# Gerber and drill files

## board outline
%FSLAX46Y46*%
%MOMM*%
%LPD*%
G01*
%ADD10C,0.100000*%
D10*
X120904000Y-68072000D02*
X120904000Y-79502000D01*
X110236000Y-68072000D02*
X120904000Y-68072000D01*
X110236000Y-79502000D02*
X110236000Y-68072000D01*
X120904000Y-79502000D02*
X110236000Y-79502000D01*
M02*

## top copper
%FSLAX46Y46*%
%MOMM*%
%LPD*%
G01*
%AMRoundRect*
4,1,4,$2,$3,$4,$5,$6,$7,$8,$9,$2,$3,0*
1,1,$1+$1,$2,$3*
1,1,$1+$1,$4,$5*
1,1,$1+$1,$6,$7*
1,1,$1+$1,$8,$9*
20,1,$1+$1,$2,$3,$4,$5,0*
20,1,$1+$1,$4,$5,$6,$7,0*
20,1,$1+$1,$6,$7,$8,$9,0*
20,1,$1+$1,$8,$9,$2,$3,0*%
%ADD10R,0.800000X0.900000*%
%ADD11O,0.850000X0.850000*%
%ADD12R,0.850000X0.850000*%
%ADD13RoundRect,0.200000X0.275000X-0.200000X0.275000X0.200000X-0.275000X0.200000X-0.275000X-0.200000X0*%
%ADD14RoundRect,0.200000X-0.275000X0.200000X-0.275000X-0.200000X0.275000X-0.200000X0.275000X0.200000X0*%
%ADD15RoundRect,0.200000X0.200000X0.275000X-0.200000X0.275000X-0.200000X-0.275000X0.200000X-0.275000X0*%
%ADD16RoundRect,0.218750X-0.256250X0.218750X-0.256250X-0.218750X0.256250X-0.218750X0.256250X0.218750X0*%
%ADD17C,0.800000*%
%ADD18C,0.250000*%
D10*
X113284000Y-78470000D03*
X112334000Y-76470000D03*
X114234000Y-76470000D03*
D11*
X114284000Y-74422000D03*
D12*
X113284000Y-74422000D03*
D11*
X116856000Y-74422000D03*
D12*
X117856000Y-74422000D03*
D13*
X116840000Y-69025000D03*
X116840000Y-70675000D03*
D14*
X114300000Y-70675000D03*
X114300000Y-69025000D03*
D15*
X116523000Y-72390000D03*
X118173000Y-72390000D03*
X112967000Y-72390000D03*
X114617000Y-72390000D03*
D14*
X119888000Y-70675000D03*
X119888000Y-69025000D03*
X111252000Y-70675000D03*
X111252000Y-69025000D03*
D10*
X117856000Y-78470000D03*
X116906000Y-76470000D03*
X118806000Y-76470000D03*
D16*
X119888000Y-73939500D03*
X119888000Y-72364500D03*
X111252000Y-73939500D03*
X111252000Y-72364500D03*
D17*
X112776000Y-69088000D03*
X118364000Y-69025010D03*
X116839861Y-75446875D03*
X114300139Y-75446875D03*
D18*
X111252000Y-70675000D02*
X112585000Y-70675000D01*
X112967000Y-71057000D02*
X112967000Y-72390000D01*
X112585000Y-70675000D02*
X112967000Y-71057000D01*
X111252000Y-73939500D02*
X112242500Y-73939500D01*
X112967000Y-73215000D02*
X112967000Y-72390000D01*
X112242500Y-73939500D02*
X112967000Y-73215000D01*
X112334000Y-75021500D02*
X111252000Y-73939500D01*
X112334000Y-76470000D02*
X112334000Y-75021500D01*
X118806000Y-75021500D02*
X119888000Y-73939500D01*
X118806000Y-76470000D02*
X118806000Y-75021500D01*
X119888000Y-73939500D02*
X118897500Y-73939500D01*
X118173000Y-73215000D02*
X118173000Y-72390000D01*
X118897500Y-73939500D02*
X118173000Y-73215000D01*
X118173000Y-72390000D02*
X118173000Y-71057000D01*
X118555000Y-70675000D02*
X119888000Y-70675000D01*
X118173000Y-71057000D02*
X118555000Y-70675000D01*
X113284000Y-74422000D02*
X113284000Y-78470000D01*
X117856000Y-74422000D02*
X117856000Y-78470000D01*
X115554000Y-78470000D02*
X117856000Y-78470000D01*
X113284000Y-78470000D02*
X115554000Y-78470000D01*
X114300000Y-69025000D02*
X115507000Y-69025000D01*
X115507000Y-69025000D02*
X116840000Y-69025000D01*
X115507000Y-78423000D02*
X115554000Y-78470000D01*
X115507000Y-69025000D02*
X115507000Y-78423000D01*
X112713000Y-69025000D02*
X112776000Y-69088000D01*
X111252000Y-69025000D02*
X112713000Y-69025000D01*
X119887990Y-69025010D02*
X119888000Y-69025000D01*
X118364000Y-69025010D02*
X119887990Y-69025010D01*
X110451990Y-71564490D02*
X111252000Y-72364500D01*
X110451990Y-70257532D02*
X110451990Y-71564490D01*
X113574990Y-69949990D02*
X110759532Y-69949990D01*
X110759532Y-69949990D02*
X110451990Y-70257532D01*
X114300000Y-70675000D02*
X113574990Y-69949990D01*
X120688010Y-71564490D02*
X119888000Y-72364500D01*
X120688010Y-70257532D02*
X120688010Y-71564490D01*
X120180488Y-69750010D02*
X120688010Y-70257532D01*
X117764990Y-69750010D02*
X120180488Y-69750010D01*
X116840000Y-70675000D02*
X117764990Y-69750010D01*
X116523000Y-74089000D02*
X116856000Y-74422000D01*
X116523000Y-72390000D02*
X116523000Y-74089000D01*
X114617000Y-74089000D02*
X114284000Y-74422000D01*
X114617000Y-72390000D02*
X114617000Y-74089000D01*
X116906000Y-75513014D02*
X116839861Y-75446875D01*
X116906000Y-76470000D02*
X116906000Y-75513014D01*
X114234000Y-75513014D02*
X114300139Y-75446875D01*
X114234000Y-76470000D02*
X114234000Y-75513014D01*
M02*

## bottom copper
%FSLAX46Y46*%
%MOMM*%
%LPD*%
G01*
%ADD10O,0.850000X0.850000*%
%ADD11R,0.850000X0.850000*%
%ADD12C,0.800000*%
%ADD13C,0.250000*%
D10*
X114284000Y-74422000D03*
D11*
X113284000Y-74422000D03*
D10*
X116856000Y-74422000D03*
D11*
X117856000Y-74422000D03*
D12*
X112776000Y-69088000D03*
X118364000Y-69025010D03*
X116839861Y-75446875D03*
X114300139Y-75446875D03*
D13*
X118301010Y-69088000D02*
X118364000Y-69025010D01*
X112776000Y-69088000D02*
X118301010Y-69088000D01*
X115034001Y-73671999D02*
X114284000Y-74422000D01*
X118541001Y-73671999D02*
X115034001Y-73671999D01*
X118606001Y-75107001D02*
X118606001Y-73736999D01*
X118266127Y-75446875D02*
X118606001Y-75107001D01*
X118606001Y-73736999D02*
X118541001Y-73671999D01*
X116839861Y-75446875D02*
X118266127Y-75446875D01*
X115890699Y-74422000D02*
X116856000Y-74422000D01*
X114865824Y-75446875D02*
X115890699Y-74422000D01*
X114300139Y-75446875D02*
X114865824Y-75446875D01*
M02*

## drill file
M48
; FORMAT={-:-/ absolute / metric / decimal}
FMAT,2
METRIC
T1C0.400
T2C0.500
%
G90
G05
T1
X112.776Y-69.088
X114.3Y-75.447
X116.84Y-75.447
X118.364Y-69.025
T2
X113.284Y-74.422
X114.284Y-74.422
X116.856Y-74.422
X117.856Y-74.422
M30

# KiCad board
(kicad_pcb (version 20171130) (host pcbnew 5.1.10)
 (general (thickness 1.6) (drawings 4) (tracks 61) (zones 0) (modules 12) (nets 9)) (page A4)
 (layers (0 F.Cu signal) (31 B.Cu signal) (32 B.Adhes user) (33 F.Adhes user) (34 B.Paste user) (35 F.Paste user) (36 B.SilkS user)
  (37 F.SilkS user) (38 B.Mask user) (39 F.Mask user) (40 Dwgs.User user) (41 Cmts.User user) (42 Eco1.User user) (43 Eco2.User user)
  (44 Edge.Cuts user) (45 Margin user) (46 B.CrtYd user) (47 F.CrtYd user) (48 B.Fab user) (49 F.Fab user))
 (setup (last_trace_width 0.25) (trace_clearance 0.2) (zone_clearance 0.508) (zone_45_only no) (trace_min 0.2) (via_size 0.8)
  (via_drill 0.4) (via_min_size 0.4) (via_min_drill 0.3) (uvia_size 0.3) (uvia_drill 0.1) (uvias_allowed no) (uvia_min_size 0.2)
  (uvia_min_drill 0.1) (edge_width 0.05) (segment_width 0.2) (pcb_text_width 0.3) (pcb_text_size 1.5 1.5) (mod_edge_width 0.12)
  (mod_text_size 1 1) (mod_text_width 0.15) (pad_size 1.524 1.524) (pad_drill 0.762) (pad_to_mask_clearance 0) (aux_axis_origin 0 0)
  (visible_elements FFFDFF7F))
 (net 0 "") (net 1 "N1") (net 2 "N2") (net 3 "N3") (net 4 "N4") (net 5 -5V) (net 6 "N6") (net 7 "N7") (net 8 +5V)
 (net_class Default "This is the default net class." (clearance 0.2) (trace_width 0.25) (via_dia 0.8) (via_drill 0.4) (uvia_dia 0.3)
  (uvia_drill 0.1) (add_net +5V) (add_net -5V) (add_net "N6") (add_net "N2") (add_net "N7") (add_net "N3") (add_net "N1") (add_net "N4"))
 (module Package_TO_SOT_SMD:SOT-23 (layer F.Cu) (at 113.284 77.47 270)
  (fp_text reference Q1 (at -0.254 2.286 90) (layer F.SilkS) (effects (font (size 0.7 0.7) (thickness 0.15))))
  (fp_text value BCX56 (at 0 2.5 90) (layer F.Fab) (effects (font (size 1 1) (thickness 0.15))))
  (pad 3 smd rect (at 1 0 270) (size 0.9 0.8) (layers F.Cu F.Paste F.Mask) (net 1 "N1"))
  (pad 2 smd rect (at -1 0.95 270) (size 0.9 0.8) (layers F.Cu F.Paste F.Mask) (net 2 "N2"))
  (pad 1 smd rect (at -1 -0.95 270) (size 0.9 0.8) (layers F.Cu F.Paste F.Mask) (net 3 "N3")))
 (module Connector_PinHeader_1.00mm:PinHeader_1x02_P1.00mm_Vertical (layer F.Cu) (at 113.284 74.422 90)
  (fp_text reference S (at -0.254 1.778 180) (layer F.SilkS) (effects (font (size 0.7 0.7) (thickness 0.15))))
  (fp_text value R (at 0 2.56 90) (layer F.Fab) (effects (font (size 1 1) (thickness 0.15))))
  (pad 2 thru_hole oval (at 0 1 90) (size 0.85 0.85) (drill 0.5) (layers *.Cu *.Mask) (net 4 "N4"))
  (pad 1 thru_hole rect (at 0 0 90) (size 0.85 0.85) (drill 0.5) (layers *.Cu *.Mask) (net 1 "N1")))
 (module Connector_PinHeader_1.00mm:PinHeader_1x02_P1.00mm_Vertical (layer F.Cu) (at 117.856 74.422 270)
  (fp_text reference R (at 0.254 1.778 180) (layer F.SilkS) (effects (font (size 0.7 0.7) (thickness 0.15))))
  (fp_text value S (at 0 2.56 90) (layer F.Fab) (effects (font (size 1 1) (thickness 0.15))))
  (pad 2 thru_hole oval (at 0 1 270) (size 0.85 0.85) (drill 0.5) (layers *.Cu *.Mask) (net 3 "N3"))
  (pad 1 thru_hole rect (at 0 0 270) (size 0.85 0.85) (drill 0.5) (layers *.Cu *.Mask) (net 1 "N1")))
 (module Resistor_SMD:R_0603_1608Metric (layer F.Cu) (at 116.84 69.85 90)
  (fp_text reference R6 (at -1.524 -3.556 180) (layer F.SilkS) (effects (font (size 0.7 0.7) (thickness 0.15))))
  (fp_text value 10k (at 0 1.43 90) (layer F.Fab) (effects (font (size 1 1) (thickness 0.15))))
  (pad 2 smd roundrect (at 0.825 0 90) (size 0.8 0.95) (layers F.Cu F.Paste F.Mask) (roundrect_rratio 0.25) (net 1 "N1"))
  (pad 1 smd roundrect (at -0.825 0 90) (size 0.8 0.95) (layers F.Cu F.Paste F.Mask) (roundrect_rratio 0.25) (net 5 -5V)))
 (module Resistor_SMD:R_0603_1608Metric (layer F.Cu) (at 114.3 69.85 270)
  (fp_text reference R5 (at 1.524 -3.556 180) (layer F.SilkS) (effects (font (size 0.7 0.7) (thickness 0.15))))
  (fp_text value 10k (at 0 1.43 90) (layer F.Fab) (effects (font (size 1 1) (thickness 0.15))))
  (pad 2 smd roundrect (at 0.825 0 270) (size 0.8 0.95) (layers F.Cu F.Paste F.Mask) (roundrect_rratio 0.25) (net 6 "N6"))
  (pad 1 smd roundrect (at -0.825 0 270) (size 0.8 0.95) (layers F.Cu F.Paste F.Mask) (roundrect_rratio 0.25) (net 1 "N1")))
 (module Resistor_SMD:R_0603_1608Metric (layer F.Cu) (at 117.348 72.39 180)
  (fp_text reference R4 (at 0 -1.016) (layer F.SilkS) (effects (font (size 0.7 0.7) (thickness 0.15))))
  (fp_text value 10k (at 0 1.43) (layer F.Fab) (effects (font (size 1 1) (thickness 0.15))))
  (pad 2 smd roundrect (at 0.825 0 180) (size 0.8 0.95) (layers F.Cu F.Paste F.Mask) (roundrect_rratio 0.25) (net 3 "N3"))
  (pad 1 smd roundrect (at -0.825 0 180) (size 0.8 0.95) (layers F.Cu F.Paste F.Mask) (roundrect_rratio 0.25) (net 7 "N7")))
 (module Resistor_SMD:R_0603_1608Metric (layer F.Cu) (at 113.792 72.39 180)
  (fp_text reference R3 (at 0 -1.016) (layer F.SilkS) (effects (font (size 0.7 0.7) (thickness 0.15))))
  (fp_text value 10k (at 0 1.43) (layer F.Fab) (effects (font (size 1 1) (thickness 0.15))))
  (pad 2 smd roundrect (at 0.825 0 180) (size 0.8 0.95) (layers F.Cu F.Paste F.Mask) (roundrect_rratio 0.25) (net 2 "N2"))
  (pad 1 smd roundrect (at -0.825 0 180) (size 0.8 0.95) (layers F.Cu F.Paste F.Mask) (roundrect_rratio 0.25) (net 4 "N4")))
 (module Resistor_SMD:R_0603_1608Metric (layer F.Cu) (at 119.888 69.85 270)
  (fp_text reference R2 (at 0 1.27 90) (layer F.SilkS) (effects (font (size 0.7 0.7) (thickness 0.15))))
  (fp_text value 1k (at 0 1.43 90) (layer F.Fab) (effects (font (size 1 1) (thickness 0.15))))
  (pad 2 smd roundrect (at 0.825 0 270) (size 0.8 0.95) (layers F.Cu F.Paste F.Mask) (roundrect_rratio 0.25) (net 7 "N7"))
  (pad 1 smd roundrect (at -0.825 0 270) (size 0.8 0.95) (layers F.Cu F.Paste F.Mask) (roundrect_rratio 0.25) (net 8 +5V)))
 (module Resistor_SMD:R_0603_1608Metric (layer F.Cu) (at 111.252 69.85 270)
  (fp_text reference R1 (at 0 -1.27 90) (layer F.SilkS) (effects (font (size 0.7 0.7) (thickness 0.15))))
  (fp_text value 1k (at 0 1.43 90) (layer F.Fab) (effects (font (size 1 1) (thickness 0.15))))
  (pad 2 smd roundrect (at 0.825 0 270) (size 0.8 0.95) (layers F.Cu F.Paste F.Mask) (roundrect_rratio 0.25) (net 2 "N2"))
  (pad 1 smd roundrect (at -0.825 0 270) (size 0.8 0.95) (layers F.Cu F.Paste F.Mask) (roundrect_rratio 0.25) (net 8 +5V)))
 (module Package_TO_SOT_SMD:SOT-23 (layer F.Cu) (at 117.856 77.47 270)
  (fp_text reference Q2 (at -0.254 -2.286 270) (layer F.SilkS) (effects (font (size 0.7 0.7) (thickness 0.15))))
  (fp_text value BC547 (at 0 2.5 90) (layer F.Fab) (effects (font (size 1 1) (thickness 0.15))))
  (pad 3 smd rect (at 1 0 270) (size 0.9 0.8) (layers F.Cu F.Paste F.Mask) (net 1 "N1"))
  (pad 2 smd rect (at -1 0.95 270) (size 0.9 0.8) (layers F.Cu F.Paste F.Mask) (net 4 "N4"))
  (pad 1 smd rect (at -1 -0.95 270) (size 0.9 0.8) (layers F.Cu F.Paste F.Mask) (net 7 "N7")))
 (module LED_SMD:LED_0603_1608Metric (layer F.Cu) (at 119.888 73.152 270)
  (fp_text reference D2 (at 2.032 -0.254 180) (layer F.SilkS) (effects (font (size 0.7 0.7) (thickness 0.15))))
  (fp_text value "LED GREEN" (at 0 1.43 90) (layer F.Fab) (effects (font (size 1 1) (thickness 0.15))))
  (pad 2 smd roundrect (at 0.7875 0 270) (size 0.875 0.95) (layers F.Cu F.Paste F.Mask) (roundrect_rratio 0.25) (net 7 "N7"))
  (pad 1 smd roundrect (at -0.7875 0 270) (size 0.875 0.95) (layers F.Cu F.Paste F.Mask) (roundrect_rratio 0.25) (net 5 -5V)))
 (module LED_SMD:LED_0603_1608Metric (layer F.Cu) (at 111.252 73.152 270)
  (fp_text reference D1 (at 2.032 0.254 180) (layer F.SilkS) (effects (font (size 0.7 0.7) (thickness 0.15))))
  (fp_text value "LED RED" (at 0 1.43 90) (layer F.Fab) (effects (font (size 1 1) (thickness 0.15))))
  (pad 2 smd roundrect (at 0.7875 0 270) (size 0.875 0.95) (layers F.Cu F.Paste F.Mask) (roundrect_rratio 0.25) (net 2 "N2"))
  (pad 1 smd roundrect (at -0.7875 0 270) (size 0.875 0.95) (layers F.Cu F.Paste F.Mask) (roundrect_rratio 0.25) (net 6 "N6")))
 (gr_line (start 120.904 68.072) (end 120.904 79.502) (layer Edge.Cuts) (width 0.1))
 (gr_line (start 110.236 68.072) (end 120.904 68.072) (layer Edge.Cuts) (width 0.1))
 (gr_line (start 110.236 79.502) (end 110.236 68.072) (layer Edge.Cuts) (width 0.1))
 (gr_line (start 120.904 79.502) (end 110.236 79.502) (layer Edge.Cuts) (width 0.1))
 (segment (start 111.252 70.675) (end 112.585 70.675) (width 0.25) (layer F.Cu) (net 2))
 (segment (start 112.967 71.057) (end 112.967 72.39) (width 0.25) (layer F.Cu) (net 2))
 (segment (start 112.585 70.675) (end 112.967 71.057) (width 0.25) (layer F.Cu) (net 2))
 (segment (start 111.252 73.9395) (end 112.2425 73.9395) (width 0.25) (layer F.Cu) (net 2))
 (segment (start 112.967 73.215) (end 112.967 72.39) (width 0.25) (layer F.Cu) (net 2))
 (segment (start 112.2425 73.9395) (end 112.967 73.215) (width 0.25) (layer F.Cu) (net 2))
 (segment (start 112.334 75.0215) (end 111.252 73.9395) (width 0.25) (layer F.Cu) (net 2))
 (segment (start 112.334 76.47) (end 112.334 75.0215) (width 0.25) (layer F.Cu) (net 2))
 (segment (start 118.806 75.0215) (end 119.888 73.9395) (width 0.25) (layer F.Cu) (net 7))
 (segment (start 118.806 76.47) (end 118.806 75.0215) (width 0.25) (layer F.Cu) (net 7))
 (segment (start 119.888 73.9395) (end 118.8975 73.9395) (width 0.25) (layer F.Cu) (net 7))
 (segment (start 118.173 73.215) (end 118.173 72.39) (width 0.25) (layer F.Cu) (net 7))
 (segment (start 118.8975 73.9395) (end 118.173 73.215) (width 0.25) (layer F.Cu) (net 7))
 (segment (start 118.173 72.39) (end 118.173 71.057) (width 0.25) (layer F.Cu) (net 7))
 (segment (start 118.555 70.675) (end 119.888 70.675) (width 0.25) (layer F.Cu) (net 7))
 (segment (start 118.173 71.057) (end 118.555 70.675) (width 0.25) (layer F.Cu) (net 7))
 (segment (start 113.284 74.422) (end 113.284 78.47) (width 0.25) (layer F.Cu) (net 1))
 (segment (start 117.856 74.422) (end 117.856 78.47) (width 0.25) (layer F.Cu) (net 1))
 (segment (start 115.554 78.47) (end 117.856 78.47) (width 0.25) (layer F.Cu) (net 1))
 (segment (start 113.284 78.47) (end 115.554 78.47) (width 0.25) (layer F.Cu) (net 1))
 (segment (start 114.3 69.025) (end 115.507 69.025) (width 0.25) (layer F.Cu) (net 1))
 (segment (start 115.507 69.025) (end 116.84 69.025) (width 0.25) (layer F.Cu) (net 1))
 (segment (start 115.507 78.423) (end 115.554 78.47) (width 0.25) (layer F.Cu) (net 1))
 (segment (start 115.507 69.025) (end 115.507 78.423) (width 0.25) (layer F.Cu) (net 1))
 (via (at 112.776 69.088) (size 0.8) (drill 0.4) (layers F.Cu B.Cu) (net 8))
 (segment (start 112.713 69.025) (end 112.776 69.088) (width 0.25) (layer F.Cu) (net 8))
 (segment (start 111.252 69.025) (end 112.713 69.025) (width 0.25) (layer F.Cu) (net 8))
 (via (at 118.364 69.02501) (size 0.8) (drill 0.4) (layers F.Cu B.Cu) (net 8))
 (segment (start 118.30101 69.088) (end 118.364 69.02501) (width 0.25) (layer B.Cu) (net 8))
 (segment (start 112.776 69.088) (end 118.30101 69.088) (width 0.25) (layer B.Cu) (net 8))
 (segment (start 119.88799 69.02501) (end 119.888 69.025) (width 0.25) (layer F.Cu) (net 8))
 (segment (start 118.364 69.02501) (end 119.88799 69.02501) (width 0.25) (layer F.Cu) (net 8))
 (segment (start 110.45199 71.56449) (end 111.252 72.3645) (width 0.25) (layer F.Cu) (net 6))
 (segment (start 110.45199 70.257532) (end 110.45199 71.56449) (width 0.25) (layer F.Cu) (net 6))
 (segment (start 113.57499 69.94999) (end 110.759532 69.94999) (width 0.25) (layer F.Cu) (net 6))
 (segment (start 110.759532 69.94999) (end 110.45199 70.257532) (width 0.25) (layer F.Cu) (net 6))
 (segment (start 114.3 70.675) (end 113.57499 69.94999) (width 0.25) (layer F.Cu) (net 6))
 (segment (start 120.68801 71.56449) (end 119.888 72.3645) (width 0.25) (layer F.Cu) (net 5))
 (segment (start 120.68801 70.257532) (end 120.68801 71.56449) (width 0.25) (layer F.Cu) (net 5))
 (segment (start 120.180488 69.75001) (end 120.68801 70.257532) (width 0.25) (layer F.Cu) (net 5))
 (segment (start 117.76499 69.75001) (end 120.180488 69.75001) (width 0.25) (layer F.Cu) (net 5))
 (segment (start 116.84 70.675) (end 117.76499 69.75001) (width 0.25) (layer F.Cu) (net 5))
 (segment (start 116.523 74.089) (end 116.856 74.422) (width 0.25) (layer F.Cu) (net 3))
 (segment (start 116.523 72.39) (end 116.523 74.089) (width 0.25) (layer F.Cu) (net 3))
 (segment (start 114.617 74.089) (end 114.284 74.422) (width 0.25) (layer F.Cu) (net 4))
 (segment (start 114.617 72.39) (end 114.617 74.089) (width 0.25) (layer F.Cu) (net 4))
 (via (at 116.839861 75.446875) (size 0.8) (drill 0.4) (layers F.Cu B.Cu) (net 4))
 (segment (start 116.906 75.513014) (end 116.839861 75.446875) (width 0.25) (layer F.Cu) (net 4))
 (segment (start 116.906 76.47) (end 116.906 75.513014) (width 0.25) (layer F.Cu) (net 4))
 (segment (start 115.034001 73.671999) (end 114.284 74.422) (width 0.25) (layer B.Cu) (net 4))
 (segment (start 118.541001 73.671999) (end 115.034001 73.671999) (width 0.25) (layer B.Cu) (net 4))
 (segment (start 118.606001 75.107001) (end 118.606001 73.736999) (width 0.25) (layer B.Cu) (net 4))
 (segment (start 118.266127 75.446875) (end 118.606001 75.107001) (width 0.25) (layer B.Cu) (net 4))
 (segment (start 118.606001 73.736999) (end 118.541001 73.671999) (width 0.25) (layer B.Cu) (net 4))
 (segment (start 116.839861 75.446875) (end 118.266127 75.446875) (width 0.25) (layer B.Cu) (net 4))
 (via (at 114.300139 75.446875) (size 0.8) (drill 0.4) (layers F.Cu B.Cu) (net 3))
 (segment (start 114.234 75.513014) (end 114.300139 75.446875) (width 0.25) (layer F.Cu) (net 3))
 (segment (start 114.234 76.47) (end 114.234 75.513014) (width 0.25) (layer F.Cu) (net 3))
 (segment (start 115.890699 74.422) (end 116.856 74.422) (width 0.25) (layer B.Cu) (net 3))
 (segment (start 114.865824 75.446875) (end 115.890699 74.422) (width 0.25) (layer B.Cu) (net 3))
 (segment (start 114.300139 75.446875) (end 114.865824 75.446875) (width 0.25) (layer B.Cu) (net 3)))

